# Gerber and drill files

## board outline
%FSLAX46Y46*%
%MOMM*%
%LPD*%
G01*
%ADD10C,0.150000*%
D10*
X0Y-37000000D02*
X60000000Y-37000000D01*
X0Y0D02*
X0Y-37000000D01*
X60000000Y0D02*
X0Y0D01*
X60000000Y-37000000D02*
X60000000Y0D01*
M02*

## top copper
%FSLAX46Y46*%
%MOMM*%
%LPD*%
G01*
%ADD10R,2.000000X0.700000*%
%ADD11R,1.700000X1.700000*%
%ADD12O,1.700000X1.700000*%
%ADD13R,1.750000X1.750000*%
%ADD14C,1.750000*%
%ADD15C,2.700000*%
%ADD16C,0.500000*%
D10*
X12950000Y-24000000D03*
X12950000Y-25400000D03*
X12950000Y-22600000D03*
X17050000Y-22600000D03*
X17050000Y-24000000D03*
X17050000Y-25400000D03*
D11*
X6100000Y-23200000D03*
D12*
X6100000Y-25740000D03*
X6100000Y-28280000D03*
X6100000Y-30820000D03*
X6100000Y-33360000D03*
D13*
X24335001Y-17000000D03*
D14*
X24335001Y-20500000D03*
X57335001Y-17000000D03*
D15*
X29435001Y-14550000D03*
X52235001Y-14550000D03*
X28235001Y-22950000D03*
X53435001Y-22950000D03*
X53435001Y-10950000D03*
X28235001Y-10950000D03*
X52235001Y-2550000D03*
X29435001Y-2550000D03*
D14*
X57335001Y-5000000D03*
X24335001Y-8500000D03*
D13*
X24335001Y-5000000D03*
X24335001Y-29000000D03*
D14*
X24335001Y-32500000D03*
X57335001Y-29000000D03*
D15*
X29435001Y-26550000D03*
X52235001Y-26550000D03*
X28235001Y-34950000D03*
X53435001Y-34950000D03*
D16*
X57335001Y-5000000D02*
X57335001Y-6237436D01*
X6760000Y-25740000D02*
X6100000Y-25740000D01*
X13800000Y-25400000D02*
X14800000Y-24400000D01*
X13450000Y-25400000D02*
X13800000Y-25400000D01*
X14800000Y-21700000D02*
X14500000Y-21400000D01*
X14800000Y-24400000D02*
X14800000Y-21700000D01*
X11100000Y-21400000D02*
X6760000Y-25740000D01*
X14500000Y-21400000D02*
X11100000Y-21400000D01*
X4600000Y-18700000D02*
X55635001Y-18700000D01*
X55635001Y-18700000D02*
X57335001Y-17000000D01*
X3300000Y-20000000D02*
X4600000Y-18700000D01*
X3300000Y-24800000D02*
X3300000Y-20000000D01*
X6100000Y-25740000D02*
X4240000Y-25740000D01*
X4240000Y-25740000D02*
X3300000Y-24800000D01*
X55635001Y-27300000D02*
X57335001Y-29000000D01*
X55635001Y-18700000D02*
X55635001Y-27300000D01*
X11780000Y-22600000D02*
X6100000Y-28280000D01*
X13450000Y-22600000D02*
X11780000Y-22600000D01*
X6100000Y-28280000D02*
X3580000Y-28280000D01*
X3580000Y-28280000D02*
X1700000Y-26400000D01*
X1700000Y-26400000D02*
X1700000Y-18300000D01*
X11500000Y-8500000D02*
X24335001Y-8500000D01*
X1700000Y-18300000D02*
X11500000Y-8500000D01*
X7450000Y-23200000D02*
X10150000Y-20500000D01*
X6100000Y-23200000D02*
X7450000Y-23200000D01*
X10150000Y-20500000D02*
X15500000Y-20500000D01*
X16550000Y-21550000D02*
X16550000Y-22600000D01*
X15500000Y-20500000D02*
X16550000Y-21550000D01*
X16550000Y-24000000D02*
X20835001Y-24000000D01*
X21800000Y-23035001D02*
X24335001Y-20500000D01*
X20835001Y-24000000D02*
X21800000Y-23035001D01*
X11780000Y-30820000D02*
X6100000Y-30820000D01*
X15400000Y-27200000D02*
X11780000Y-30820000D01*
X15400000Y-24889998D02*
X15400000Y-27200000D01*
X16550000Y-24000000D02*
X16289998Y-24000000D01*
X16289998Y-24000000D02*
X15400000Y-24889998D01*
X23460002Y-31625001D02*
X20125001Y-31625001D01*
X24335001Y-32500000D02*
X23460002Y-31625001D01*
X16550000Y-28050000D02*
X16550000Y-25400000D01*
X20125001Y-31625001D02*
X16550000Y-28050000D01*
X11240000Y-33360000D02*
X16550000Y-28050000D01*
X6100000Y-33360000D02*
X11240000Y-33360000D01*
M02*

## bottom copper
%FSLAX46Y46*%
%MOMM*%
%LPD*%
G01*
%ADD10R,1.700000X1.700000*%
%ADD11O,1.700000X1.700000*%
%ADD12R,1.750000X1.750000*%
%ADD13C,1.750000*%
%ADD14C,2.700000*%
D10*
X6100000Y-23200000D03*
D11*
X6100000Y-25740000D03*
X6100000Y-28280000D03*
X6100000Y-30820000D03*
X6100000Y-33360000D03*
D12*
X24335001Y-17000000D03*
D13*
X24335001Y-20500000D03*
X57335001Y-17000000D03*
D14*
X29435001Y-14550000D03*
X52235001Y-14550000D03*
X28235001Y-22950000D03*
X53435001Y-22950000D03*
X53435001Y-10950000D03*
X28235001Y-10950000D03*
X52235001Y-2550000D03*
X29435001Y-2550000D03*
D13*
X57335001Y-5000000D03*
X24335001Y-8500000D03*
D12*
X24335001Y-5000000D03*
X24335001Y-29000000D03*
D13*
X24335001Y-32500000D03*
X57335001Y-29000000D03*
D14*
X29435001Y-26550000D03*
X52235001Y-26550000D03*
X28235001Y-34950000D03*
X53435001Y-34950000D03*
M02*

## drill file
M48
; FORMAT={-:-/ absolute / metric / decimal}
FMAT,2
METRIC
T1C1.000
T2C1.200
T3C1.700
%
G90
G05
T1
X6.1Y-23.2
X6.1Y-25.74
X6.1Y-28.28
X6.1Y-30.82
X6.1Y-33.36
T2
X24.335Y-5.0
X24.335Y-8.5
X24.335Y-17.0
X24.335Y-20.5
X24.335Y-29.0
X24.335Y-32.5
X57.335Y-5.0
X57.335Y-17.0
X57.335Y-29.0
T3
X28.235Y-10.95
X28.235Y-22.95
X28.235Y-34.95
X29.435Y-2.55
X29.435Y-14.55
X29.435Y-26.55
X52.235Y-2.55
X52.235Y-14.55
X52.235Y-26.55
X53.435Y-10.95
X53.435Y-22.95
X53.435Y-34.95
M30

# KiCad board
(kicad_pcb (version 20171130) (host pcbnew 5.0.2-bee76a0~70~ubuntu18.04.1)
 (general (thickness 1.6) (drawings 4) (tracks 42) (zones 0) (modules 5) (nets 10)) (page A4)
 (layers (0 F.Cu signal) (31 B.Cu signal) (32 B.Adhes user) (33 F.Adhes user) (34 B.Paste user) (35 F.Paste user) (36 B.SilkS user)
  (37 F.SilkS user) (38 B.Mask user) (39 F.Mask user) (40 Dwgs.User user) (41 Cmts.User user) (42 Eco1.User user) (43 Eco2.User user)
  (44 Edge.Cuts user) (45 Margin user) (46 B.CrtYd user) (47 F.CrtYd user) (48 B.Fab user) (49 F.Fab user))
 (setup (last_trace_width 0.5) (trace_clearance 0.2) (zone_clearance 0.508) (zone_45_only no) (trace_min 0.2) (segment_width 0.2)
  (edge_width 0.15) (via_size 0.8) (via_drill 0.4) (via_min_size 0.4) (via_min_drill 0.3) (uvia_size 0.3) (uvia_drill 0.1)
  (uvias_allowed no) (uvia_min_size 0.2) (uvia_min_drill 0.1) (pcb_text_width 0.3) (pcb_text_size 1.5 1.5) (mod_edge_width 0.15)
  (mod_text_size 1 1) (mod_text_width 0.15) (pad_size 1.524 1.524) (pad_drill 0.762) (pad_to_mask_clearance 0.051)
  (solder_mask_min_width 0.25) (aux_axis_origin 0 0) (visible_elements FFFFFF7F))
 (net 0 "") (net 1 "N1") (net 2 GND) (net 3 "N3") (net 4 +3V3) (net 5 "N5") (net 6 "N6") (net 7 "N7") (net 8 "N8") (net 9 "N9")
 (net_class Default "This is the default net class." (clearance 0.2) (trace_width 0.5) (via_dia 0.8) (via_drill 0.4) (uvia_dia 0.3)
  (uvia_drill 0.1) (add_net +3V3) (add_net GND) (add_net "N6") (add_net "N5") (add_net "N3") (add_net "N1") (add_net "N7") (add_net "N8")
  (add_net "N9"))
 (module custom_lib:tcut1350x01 (layer F.Cu) (at 15 24 180)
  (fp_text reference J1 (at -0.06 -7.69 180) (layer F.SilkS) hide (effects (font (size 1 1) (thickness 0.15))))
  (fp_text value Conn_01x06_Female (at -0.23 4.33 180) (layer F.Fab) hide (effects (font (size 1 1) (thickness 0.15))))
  (pad 5 smd rect (at 1.55 0 180) (size 2 0.7) (drill (offset 0.5 0)) (layers F.Cu F.Paste F.Mask) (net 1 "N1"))
  (pad 6 smd rect (at 1.55 -1.4 180) (size 2 0.7) (drill (offset 0.5 0)) (layers F.Cu F.Paste F.Mask) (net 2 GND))
  (pad 4 smd rect (at 1.55 1.4 180) (size 2 0.7) (drill (offset 0.5 0)) (layers F.Cu F.Paste F.Mask) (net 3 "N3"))
  (pad 3 smd rect (at -1.55 1.4 180) (size 2 0.7) (drill (offset -0.5 0)) (layers F.Cu F.Paste F.Mask) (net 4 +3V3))
  (pad 2 smd rect (at -1.55 0 180) (size 2 0.7) (drill (offset -0.5 0)) (layers F.Cu F.Paste F.Mask) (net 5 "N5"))
  (pad 1 smd rect (at -1.55 -1.4 180) (size 2 0.7) (drill (offset -0.5 0)) (layers F.Cu F.Paste F.Mask) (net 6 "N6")))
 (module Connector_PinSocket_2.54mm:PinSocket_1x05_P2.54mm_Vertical (layer F.Cu) (at 6.1 23.2)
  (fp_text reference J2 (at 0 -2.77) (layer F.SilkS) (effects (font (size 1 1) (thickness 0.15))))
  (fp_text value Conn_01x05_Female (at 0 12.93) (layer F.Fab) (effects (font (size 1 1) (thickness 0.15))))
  (pad 1 thru_hole rect (at 0 0) (size 1.7 1.7) (drill 1) (layers *.Cu *.Mask) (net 4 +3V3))
  (pad 2 thru_hole oval (at 0 2.54) (size 1.7 1.7) (drill 1) (layers *.Cu *.Mask) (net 2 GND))
  (pad 3 thru_hole oval (at 0 5.08) (size 1.7 1.7) (drill 1) (layers *.Cu *.Mask) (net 3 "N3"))
  (pad 4 thru_hole oval (at 0 7.62) (size 1.7 1.7) (drill 1) (layers *.Cu *.Mask) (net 5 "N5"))
  (pad 5 thru_hole oval (at 0 10.16) (size 1.7 1.7) (drill 1) (layers *.Cu *.Mask) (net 6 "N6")))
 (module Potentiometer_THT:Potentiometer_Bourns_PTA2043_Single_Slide (layer F.Cu) (at 24.335001 17)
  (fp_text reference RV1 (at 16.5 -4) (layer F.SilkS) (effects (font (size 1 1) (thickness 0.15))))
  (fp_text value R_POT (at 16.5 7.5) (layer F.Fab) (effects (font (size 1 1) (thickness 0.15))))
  (pad 1 thru_hole rect (at 0 0) (size 1.75 1.75) (drill 1.2) (layers *.Cu *.Mask) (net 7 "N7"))
  (pad 2 thru_hole circle (at 0 3.5) (size 1.75 1.75) (drill 1.2) (layers *.Cu *.Mask) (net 5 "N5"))
  (pad 3 thru_hole circle (at 33 0) (size 1.75 1.75) (drill 1.2) (layers *.Cu *.Mask) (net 2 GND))
  (pad MP thru_hole circle (at 5.1 -2.45) (size 2.7 2.7) (drill 1.7) (layers *.Cu *.Mask))
  (pad MP thru_hole circle (at 27.9 -2.45) (size 2.7 2.7) (drill 1.7) (layers *.Cu *.Mask))
  (pad MP thru_hole circle (at 3.9 5.95) (size 2.7 2.7) (drill 1.7) (layers *.Cu *.Mask))
  (pad MP thru_hole circle (at 29.1 5.95) (size 2.7 2.7) (drill 1.7) (layers *.Cu *.Mask)))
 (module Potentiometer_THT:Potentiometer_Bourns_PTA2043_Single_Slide (layer F.Cu) (at 24.335001 5)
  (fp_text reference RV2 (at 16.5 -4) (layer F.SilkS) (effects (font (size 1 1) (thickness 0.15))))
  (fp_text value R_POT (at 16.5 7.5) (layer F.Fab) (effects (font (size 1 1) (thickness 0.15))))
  (pad MP thru_hole circle (at 29.1 5.95) (size 2.7 2.7) (drill 1.7) (layers *.Cu *.Mask))
  (pad MP thru_hole circle (at 3.9 5.95) (size 2.7 2.7) (drill 1.7) (layers *.Cu *.Mask))
  (pad MP thru_hole circle (at 27.9 -2.45) (size 2.7 2.7) (drill 1.7) (layers *.Cu *.Mask))
  (pad MP thru_hole circle (at 5.1 -2.45) (size 2.7 2.7) (drill 1.7) (layers *.Cu *.Mask))
  (pad 3 thru_hole circle (at 33 0) (size 1.75 1.75) (drill 1.2) (layers *.Cu *.Mask) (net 4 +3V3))
  (pad 2 thru_hole circle (at 0 3.5) (size 1.75 1.75) (drill 1.2) (layers *.Cu *.Mask) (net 3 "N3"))
  (pad 1 thru_hole rect (at 0 0) (size 1.75 1.75) (drill 1.2) (layers *.Cu *.Mask) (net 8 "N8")))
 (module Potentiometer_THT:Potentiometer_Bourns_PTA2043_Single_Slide (layer F.Cu) (at 24.335001 29)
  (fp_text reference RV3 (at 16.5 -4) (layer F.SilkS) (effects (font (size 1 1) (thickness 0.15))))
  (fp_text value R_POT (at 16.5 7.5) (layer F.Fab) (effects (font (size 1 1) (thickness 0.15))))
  (pad 1 thru_hole rect (at 0 0) (size 1.75 1.75) (drill 1.2) (layers *.Cu *.Mask) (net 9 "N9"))
  (pad 2 thru_hole circle (at 0 3.5) (size 1.75 1.75) (drill 1.2) (layers *.Cu *.Mask) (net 6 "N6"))
  (pad 3 thru_hole circle (at 33 0) (size 1.75 1.75) (drill 1.2) (layers *.Cu *.Mask) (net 2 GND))
  (pad MP thru_hole circle (at 5.1 -2.45) (size 2.7 2.7) (drill 1.7) (layers *.Cu *.Mask))
  (pad MP thru_hole circle (at 27.9 -2.45) (size 2.7 2.7) (drill 1.7) (layers *.Cu *.Mask))
  (pad MP thru_hole circle (at 3.9 5.95) (size 2.7 2.7) (drill 1.7) (layers *.Cu *.Mask))
  (pad MP thru_hole circle (at 29.1 5.95) (size 2.7 2.7) (drill 1.7) (layers *.Cu *.Mask)))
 (gr_line (start 0 37) (end 60 37) (layer Edge.Cuts) (width 0.15))
 (gr_line (start 0 0) (end 0 37) (layer Edge.Cuts) (width 0.15))
 (gr_line (start 60 0) (end 0 0) (layer Edge.Cuts) (width 0.15))
 (gr_line (start 60 37) (end 60 0) (layer Edge.Cuts) (width 0.15))
 (segment (start 57.335001 5) (end 57.335001 6.237436) (width 0.5) (layer F.Cu) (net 4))
 (segment (start 6.76 25.74) (end 6.1 25.74) (width 0.5) (layer F.Cu) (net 2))
 (segment (start 13.8 25.4) (end 14.8 24.4) (width 0.5) (layer F.Cu) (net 2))
 (segment (start 13.45 25.4) (end 13.8 25.4) (width 0.5) (layer F.Cu) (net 2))
 (segment (start 14.8 21.7) (end 14.5 21.4) (width 0.5) (layer F.Cu) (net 2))
 (segment (start 14.8 24.4) (end 14.8 21.7) (width 0.5) (layer F.Cu) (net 2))
 (segment (start 11.1 21.4) (end 6.76 25.74) (width 0.5) (layer F.Cu) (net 2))
 (segment (start 14.5 21.4) (end 11.1 21.4) (width 0.5) (layer F.Cu) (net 2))
 (segment (start 4.6 18.7) (end 55.635001 18.7) (width 0.5) (layer F.Cu) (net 2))
 (segment (start 55.635001 18.7) (end 57.335001 17) (width 0.5) (layer F.Cu) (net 2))
 (segment (start 3.3 20) (end 4.6 18.7) (width 0.5) (layer F.Cu) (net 2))
 (segment (start 3.3 24.8) (end 3.3 20) (width 0.5) (layer F.Cu) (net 2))
 (segment (start 6.1 25.74) (end 4.24 25.74) (width 0.5) (layer F.Cu) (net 2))
 (segment (start 4.24 25.74) (end 3.3 24.8) (width 0.5) (layer F.Cu) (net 2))
 (segment (start 55.635001 27.3) (end 57.335001 29) (width 0.5) (layer F.Cu) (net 2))
 (segment (start 55.635001 18.7) (end 55.635001 27.3) (width 0.5) (layer F.Cu) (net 2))
 (segment (start 11.78 22.6) (end 6.1 28.28) (width 0.5) (layer F.Cu) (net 3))
 (segment (start 13.45 22.6) (end 11.78 22.6) (width 0.5) (layer F.Cu) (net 3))
 (segment (start 6.1 28.28) (end 3.58 28.28) (width 0.5) (layer F.Cu) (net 3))
 (segment (start 3.58 28.28) (end 1.7 26.4) (width 0.5) (layer F.Cu) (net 3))
 (segment (start 1.7 26.4) (end 1.7 18.3) (width 0.5) (layer F.Cu) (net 3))
 (segment (start 11.5 8.5) (end 24.335001 8.5) (width 0.5) (layer F.Cu) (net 3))
 (segment (start 1.7 18.3) (end 11.5 8.5) (width 0.5) (layer F.Cu) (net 3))
 (segment (start 7.45 23.2) (end 10.15 20.5) (width 0.5) (layer F.Cu) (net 4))
 (segment (start 6.1 23.2) (end 7.45 23.2) (width 0.5) (layer F.Cu) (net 4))
 (segment (start 10.15 20.5) (end 15.5 20.5) (width 0.5) (layer F.Cu) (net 4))
 (segment (start 16.55 21.55) (end 16.55 22.6) (width 0.5) (layer F.Cu) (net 4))
 (segment (start 15.5 20.5) (end 16.55 21.55) (width 0.5) (layer F.Cu) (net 4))
 (segment (start 16.55 24) (end 20.835001 24) (width 0.5) (layer F.Cu) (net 5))
 (segment (start 21.8 23.035001) (end 24.335001 20.5) (width 0.5) (layer F.Cu) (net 5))
 (segment (start 20.835001 24) (end 21.8 23.035001) (width 0.5) (layer F.Cu) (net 5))
 (segment (start 11.78 30.82) (end 6.1 30.82) (width 0.5) (layer F.Cu) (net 5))
 (segment (start 15.4 27.2) (end 11.78 30.82) (width 0.5) (layer F.Cu) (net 5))
 (segment (start 15.4 24.889998) (end 15.4 27.2) (width 0.5) (layer F.Cu) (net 5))
 (segment (start 16.55 24) (end 16.289998 24) (width 0.5) (layer F.Cu) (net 5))
 (segment (start 16.289998 24) (end 15.4 24.889998) (width 0.5) (layer F.Cu) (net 5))
 (segment (start 23.460002 31.625001) (end 20.125001 31.625001) (width 0.5) (layer F.Cu) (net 6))
 (segment (start 24.335001 32.5) (end 23.460002 31.625001) (width 0.5) (layer F.Cu) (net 6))
 (segment (start 16.55 28.05) (end 16.55 25.4) (width 0.5) (layer F.Cu) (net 6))
 (segment (start 20.125001 31.625001) (end 16.55 28.05) (width 0.5) (layer F.Cu) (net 6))
 (segment (start 11.24 33.36) (end 16.55 28.05) (width 0.5) (layer F.Cu) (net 6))
 (segment (start 6.1 33.36) (end 11.24 33.36) (width 0.5) (layer F.Cu) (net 6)))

